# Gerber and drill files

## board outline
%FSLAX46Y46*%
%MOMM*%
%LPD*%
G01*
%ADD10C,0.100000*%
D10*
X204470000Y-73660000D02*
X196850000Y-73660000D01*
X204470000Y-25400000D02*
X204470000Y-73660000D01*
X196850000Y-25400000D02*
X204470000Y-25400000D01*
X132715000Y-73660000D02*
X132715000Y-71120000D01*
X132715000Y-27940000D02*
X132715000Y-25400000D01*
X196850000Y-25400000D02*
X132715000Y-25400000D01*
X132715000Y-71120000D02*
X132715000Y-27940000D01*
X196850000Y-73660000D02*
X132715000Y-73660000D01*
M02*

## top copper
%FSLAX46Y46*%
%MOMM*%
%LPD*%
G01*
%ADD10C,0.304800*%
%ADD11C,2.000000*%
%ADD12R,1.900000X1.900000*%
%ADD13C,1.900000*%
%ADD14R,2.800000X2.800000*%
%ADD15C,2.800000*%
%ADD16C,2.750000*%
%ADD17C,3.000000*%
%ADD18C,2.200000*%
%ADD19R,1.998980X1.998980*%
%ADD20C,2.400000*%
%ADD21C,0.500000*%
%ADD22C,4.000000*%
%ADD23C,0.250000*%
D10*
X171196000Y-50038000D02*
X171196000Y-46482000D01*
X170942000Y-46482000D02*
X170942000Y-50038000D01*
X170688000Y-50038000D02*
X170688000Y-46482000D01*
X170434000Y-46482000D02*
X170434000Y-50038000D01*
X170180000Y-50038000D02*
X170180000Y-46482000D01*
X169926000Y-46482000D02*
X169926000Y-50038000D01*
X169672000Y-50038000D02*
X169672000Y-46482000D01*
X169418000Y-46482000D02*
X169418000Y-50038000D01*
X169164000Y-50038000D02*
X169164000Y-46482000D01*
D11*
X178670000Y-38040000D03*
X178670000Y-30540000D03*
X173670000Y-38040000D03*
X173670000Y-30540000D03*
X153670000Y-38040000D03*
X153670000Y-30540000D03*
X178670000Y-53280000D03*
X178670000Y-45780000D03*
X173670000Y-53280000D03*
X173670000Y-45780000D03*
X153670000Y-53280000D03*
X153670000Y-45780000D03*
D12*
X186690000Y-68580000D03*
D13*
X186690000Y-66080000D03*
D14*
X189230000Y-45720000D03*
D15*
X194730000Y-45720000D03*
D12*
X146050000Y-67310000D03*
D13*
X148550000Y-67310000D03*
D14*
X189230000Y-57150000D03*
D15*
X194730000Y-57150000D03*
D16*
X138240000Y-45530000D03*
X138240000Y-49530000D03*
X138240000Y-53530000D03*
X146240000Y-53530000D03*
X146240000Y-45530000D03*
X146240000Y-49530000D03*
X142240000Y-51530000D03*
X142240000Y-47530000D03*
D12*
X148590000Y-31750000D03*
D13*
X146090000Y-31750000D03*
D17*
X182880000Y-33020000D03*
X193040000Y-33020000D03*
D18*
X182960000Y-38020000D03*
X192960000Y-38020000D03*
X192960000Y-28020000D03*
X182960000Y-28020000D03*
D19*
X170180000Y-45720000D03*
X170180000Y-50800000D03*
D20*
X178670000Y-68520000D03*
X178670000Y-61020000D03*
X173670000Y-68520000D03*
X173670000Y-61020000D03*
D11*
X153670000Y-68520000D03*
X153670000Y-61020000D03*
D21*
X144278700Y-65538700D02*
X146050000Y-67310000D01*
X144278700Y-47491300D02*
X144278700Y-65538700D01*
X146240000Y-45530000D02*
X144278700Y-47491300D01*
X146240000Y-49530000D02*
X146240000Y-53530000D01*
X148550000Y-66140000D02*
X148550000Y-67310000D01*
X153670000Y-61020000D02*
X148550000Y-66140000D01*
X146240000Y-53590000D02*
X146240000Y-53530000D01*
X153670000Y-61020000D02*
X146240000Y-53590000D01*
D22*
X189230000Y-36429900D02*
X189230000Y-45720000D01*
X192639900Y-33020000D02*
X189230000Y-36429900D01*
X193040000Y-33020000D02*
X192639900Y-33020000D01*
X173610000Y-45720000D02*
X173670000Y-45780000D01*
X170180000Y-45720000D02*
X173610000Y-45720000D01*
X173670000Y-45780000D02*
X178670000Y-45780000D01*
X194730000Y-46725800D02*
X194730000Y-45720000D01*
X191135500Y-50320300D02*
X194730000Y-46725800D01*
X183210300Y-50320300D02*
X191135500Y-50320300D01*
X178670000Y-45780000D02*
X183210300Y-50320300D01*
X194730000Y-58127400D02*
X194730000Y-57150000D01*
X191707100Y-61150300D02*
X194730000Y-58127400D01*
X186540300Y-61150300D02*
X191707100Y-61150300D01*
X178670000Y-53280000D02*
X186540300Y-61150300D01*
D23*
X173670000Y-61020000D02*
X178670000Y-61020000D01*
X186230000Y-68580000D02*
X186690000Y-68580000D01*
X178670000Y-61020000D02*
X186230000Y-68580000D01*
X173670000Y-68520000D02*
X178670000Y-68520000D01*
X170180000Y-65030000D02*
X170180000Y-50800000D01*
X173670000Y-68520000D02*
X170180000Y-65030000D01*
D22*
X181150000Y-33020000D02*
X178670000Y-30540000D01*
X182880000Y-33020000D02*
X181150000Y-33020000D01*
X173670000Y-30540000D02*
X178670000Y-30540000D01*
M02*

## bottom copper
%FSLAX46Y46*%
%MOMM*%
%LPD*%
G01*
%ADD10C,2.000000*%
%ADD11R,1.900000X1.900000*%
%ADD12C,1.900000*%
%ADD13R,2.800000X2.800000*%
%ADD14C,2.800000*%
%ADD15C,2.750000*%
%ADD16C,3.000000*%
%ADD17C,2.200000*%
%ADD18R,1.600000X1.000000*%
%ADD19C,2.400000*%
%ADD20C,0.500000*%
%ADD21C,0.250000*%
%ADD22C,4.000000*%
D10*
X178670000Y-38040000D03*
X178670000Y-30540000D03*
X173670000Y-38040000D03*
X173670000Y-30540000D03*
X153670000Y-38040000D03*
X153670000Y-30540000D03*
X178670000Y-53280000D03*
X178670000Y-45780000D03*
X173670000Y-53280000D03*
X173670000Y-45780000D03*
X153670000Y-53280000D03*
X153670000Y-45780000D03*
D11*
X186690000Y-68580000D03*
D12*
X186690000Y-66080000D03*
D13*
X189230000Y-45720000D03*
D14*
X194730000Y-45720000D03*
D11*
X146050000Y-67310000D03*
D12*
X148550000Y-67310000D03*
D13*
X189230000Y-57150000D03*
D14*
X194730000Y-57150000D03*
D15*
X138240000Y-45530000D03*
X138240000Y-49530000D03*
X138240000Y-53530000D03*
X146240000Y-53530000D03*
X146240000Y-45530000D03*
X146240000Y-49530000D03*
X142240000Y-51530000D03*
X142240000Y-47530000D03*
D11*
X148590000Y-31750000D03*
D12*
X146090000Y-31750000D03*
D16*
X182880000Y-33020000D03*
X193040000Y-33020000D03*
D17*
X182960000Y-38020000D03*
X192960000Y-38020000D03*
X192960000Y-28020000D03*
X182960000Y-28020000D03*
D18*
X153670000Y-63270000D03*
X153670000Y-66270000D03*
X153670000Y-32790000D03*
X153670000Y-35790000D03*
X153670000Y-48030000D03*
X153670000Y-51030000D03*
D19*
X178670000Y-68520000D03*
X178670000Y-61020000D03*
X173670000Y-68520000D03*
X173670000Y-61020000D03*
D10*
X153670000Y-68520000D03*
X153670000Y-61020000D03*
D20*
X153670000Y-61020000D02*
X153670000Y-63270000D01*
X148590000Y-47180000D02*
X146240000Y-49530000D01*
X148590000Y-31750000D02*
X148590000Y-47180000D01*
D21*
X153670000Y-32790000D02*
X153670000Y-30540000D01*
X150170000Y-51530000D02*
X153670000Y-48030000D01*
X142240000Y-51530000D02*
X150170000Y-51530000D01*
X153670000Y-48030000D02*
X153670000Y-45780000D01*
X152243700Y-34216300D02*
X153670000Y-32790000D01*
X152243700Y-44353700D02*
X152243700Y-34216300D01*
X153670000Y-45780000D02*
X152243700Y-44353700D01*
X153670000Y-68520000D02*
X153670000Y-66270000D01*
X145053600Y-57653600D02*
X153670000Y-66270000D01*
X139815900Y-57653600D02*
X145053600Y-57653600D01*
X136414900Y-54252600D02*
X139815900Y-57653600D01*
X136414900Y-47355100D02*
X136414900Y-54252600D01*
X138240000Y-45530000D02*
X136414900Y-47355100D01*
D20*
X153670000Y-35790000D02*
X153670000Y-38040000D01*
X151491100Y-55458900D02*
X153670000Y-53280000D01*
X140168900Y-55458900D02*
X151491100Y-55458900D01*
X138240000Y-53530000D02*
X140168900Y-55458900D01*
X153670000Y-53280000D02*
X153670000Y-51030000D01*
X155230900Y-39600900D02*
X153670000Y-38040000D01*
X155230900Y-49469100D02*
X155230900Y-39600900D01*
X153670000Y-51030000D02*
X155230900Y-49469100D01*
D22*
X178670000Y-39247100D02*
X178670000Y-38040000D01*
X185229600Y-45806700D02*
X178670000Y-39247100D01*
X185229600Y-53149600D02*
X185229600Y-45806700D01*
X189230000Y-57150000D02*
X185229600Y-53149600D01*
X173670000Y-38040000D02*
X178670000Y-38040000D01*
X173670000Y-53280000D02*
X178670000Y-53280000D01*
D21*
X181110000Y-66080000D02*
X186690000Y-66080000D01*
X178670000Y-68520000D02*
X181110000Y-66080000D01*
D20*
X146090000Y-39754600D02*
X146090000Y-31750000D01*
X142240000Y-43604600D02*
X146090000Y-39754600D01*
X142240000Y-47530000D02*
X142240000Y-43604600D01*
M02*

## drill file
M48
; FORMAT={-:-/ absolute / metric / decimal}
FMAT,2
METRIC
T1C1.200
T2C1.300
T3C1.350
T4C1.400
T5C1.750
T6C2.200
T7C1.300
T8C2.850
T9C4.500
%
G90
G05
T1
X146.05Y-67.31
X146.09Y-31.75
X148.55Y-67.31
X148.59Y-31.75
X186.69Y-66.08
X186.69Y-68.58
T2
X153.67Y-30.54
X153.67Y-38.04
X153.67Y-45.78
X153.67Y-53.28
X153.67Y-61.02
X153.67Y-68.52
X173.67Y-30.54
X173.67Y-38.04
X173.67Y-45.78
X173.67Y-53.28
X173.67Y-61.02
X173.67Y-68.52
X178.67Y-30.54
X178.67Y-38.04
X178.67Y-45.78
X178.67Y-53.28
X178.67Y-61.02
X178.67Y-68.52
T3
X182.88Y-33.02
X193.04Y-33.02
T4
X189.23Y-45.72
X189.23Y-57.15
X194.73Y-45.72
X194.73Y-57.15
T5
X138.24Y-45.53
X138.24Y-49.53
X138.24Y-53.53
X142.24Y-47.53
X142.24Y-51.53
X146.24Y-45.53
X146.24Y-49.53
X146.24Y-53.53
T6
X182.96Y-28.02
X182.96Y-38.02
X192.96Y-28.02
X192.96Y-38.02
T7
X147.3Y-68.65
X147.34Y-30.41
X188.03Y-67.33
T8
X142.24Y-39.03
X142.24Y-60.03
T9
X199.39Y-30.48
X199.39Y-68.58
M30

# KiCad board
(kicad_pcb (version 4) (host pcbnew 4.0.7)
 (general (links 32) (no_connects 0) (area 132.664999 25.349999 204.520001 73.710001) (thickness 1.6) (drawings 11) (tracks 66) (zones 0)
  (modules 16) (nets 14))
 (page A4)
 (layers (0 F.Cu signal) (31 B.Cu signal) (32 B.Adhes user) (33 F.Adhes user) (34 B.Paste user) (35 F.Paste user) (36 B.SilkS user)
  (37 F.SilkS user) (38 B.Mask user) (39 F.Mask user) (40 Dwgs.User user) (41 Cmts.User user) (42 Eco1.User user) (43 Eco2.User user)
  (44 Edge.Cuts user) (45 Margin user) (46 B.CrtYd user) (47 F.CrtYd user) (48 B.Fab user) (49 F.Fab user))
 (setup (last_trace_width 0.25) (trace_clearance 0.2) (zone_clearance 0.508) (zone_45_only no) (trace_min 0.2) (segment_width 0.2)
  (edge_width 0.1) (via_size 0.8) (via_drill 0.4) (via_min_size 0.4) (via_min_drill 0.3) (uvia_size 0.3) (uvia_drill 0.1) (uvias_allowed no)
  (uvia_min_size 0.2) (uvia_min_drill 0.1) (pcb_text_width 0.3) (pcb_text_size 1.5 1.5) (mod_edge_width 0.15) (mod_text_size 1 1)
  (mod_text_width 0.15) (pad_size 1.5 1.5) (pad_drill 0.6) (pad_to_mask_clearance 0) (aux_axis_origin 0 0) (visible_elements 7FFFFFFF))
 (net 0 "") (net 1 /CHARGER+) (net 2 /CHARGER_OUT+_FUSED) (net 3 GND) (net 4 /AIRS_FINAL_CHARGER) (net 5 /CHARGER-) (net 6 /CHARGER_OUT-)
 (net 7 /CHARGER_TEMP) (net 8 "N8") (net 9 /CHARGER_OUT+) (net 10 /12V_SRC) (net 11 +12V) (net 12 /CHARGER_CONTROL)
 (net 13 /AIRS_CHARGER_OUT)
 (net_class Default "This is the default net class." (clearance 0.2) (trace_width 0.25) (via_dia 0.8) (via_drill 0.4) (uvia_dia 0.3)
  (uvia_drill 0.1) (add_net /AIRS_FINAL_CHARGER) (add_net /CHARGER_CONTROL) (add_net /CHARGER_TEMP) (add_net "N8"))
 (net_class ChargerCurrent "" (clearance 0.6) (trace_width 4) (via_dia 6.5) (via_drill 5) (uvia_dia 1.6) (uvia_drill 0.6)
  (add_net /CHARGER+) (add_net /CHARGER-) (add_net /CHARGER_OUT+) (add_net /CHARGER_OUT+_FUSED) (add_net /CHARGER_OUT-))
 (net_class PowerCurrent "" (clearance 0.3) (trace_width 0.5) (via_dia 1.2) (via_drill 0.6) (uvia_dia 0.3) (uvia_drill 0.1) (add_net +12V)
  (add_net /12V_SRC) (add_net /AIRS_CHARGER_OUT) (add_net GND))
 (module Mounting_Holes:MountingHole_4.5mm (layer F.Cu) (at 199.39 68.58)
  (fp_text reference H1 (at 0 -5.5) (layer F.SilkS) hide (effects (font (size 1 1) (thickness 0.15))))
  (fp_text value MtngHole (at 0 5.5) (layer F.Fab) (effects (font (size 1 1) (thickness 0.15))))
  (pad 1 np_thru_hole circle (at 0 0) (size 4.5 4.5) (drill 4.5) (layers *.Cu *.Mask)))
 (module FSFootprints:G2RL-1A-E (layer F.Cu) (at 153.67 34.29)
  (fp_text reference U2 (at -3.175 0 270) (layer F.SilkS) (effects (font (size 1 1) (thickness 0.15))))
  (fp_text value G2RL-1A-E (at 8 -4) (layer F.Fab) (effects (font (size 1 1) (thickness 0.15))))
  (pad 5 thru_hole circle (at 25 3.75) (size 2 2) (drill 1.3) (layers *.Cu *.Mask) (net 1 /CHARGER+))
  (pad 4 thru_hole circle (at 25 -3.75) (size 2 2) (drill 1.3) (layers *.Cu *.Mask) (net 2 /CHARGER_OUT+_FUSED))
  (pad 6 thru_hole circle (at 20 3.75) (size 2 2) (drill 1.3) (layers *.Cu *.Mask) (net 1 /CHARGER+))
  (pad 3 thru_hole circle (at 20 -3.75) (size 2 2) (drill 1.3) (layers *.Cu *.Mask) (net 2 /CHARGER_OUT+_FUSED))
  (pad 8 thru_hole circle (at 0 3.75) (size 2 2) (drill 1.3) (layers *.Cu *.Mask) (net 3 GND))
  (pad 1 thru_hole circle (at 0 -3.75) (size 2 2) (drill 1.3) (layers *.Cu *.Mask) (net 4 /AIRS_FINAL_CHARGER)))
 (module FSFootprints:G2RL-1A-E (layer F.Cu) (at 153.67 49.53)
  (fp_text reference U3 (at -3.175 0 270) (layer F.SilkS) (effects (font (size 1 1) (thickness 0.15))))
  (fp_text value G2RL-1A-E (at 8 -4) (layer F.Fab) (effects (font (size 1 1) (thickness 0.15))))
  (pad 5 thru_hole circle (at 25 3.75) (size 2 2) (drill 1.3) (layers *.Cu *.Mask) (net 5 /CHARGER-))
  (pad 4 thru_hole circle (at 25 -3.75) (size 2 2) (drill 1.3) (layers *.Cu *.Mask) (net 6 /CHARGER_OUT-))
  (pad 6 thru_hole circle (at 20 3.75) (size 2 2) (drill 1.3) (layers *.Cu *.Mask) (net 5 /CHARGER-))
  (pad 3 thru_hole circle (at 20 -3.75) (size 2 2) (drill 1.3) (layers *.Cu *.Mask) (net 6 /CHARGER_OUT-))
  (pad 8 thru_hole circle (at 0 3.75) (size 2 2) (drill 1.3) (layers *.Cu *.Mask) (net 3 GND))
  (pad 1 thru_hole circle (at 0 -3.75) (size 2 2) (drill 1.3) (layers *.Cu *.Mask) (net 4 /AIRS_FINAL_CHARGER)))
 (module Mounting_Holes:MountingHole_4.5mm (layer F.Cu) (at 199.39 30.48 180)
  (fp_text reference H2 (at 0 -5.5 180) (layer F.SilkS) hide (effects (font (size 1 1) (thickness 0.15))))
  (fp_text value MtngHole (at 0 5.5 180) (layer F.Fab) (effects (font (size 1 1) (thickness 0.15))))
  (pad 1 np_thru_hole circle (at 0 0 180) (size 4.5 4.5) (drill 4.5) (layers *.Cu *.Mask)))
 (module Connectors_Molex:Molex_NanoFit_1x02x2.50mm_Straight (layer F.Cu) (at 186.69 68.58 90)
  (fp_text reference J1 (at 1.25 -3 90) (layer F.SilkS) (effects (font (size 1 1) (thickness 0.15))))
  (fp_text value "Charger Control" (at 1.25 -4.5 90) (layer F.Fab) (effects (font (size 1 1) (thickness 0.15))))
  (pad 1 thru_hole rect (at 0 0 90) (size 1.9 1.9) (drill 1.2) (layers *.Cu *.Mask) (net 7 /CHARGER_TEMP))
  (pad 2 thru_hole circle (at 2.5 0 90) (size 1.9 1.9) (drill 1.2) (layers *.Cu *.Mask) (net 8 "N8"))
  (pad "" np_thru_hole circle (at 1.25 1.34 90) (size 1.3 1.3) (drill 1.3) (layers *.Cu *.Mask)))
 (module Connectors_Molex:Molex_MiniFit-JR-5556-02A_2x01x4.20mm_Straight (layer F.Cu) (at 189.23 45.72 90)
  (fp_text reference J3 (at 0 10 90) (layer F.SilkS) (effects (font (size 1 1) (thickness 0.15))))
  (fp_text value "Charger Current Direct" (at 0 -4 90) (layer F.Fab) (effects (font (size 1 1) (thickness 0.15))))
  (pad 1 thru_hole rect (at 0 0 90) (size 2.8 2.8) (drill 1.4) (layers *.Cu *.Mask) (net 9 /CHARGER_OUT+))
  (pad 2 thru_hole circle (at 0 5.5 90) (size 2.8 2.8) (drill 1.4) (layers *.Cu *.Mask) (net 6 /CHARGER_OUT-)))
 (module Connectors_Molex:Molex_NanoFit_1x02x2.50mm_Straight (layer F.Cu) (at 146.05 67.31)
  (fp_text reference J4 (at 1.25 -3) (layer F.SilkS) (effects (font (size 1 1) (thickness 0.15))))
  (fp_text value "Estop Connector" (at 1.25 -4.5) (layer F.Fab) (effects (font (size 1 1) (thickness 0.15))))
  (pad 1 thru_hole rect (at 0 0) (size 1.9 1.9) (drill 1.2) (layers *.Cu *.Mask) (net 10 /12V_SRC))
  (pad 2 thru_hole circle (at 2.5 0) (size 1.9 1.9) (drill 1.2) (layers *.Cu *.Mask) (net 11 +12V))
  (pad "" np_thru_hole circle (at 1.25 1.34) (size 1.3 1.3) (drill 1.3) (layers *.Cu *.Mask)))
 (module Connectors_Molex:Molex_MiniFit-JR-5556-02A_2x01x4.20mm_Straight (layer F.Cu) (at 189.23 57.15 90)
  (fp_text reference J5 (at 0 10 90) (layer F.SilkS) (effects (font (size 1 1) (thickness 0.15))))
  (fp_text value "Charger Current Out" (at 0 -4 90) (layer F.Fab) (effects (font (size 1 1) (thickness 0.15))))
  (pad 1 thru_hole rect (at 0 0 90) (size 2.8 2.8) (drill 1.4) (layers *.Cu *.Mask) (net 1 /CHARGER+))
  (pad 2 thru_hole circle (at 0 5.5 90) (size 2.8 2.8) (drill 1.4) (layers *.Cu *.Mask) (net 5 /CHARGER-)))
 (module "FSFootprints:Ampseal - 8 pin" (layer F.Cu) (at 142.24 49.53 270)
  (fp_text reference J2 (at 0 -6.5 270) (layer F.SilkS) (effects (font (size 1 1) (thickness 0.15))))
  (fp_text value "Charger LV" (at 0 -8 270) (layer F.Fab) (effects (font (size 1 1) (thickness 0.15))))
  (pad "" np_thru_hole circle (at -10.5 0 270) (size 2.85 2.85) (drill 2.85) (layers *.Cu *.Mask))
  (pad 6 thru_hole circle (at -4 4 270) (size 2.75 2.75) (drill 1.75) (layers *.Cu *.Mask) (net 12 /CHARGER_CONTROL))
  (pad 7 thru_hole circle (at 0 4 270) (size 2.75 2.75) (drill 1.75) (layers *.Cu *.Mask))
  (pad 8 thru_hole circle (at 4 4 270) (size 2.75 2.75) (drill 1.75) (layers *.Cu *.Mask) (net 3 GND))
  (pad 3 thru_hole circle (at 4 -4 270) (size 2.75 2.75) (drill 1.75) (layers *.Cu *.Mask) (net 11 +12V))
  (pad 1 thru_hole circle (at -4 -4 270) (size 2.75 2.75) (drill 1.75) (layers *.Cu *.Mask) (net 10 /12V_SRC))
  (pad 2 thru_hole circle (at 0 -4 270) (size 2.75 2.75) (drill 1.75) (layers *.Cu *.Mask) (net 11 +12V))
  (pad 5 thru_hole circle (at 2 0 270) (size 2.75 2.75) (drill 1.75) (layers *.Cu *.Mask) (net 4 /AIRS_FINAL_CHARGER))
  (pad 4 thru_hole circle (at -2 0 270) (size 2.75 2.75) (drill 1.75) (layers *.Cu *.Mask) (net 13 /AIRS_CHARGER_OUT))
  (pad "" np_thru_hole circle (at 10.5 0 270) (size 2.85 2.85) (drill 2.85) (layers *.Cu *.Mask)))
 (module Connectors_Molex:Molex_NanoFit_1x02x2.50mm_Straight (layer F.Cu) (at 148.59 31.75 180)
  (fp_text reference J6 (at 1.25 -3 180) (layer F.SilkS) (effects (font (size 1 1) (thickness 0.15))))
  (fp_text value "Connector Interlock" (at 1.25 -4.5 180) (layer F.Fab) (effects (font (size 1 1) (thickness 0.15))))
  (pad 1 thru_hole rect (at 0 0 180) (size 1.9 1.9) (drill 1.2) (layers *.Cu *.Mask) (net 11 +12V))
  (pad 2 thru_hole circle (at 2.5 0 180) (size 1.9 1.9) (drill 1.2) (layers *.Cu *.Mask) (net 13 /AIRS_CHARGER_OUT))
  (pad "" np_thru_hole circle (at 1.25 1.34 180) (size 1.3 1.3) (drill 1.3) (layers *.Cu *.Mask)))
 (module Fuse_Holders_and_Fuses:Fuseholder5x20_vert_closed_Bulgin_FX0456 (layer F.Cu) (at 193.04 33.02 180)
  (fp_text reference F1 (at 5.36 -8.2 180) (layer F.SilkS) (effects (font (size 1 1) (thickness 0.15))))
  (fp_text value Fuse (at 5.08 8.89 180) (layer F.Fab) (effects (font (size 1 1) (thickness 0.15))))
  (pad 2 thru_hole circle (at 10.16 0 180) (size 3 3) (drill 1.35) (layers *.Cu *.Mask) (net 2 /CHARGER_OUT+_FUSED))
  (pad 1 thru_hole circle (at 0 0 180) (size 3 3) (drill 1.35) (layers *.Cu *.Mask) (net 9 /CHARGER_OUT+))
  (pad 3 thru_hole circle (at 10.08 -5 180) (size 2.2 2.2) (drill 2.2) (layers *.Cu Dwgs.User))
  (pad 3 thru_hole circle (at 0.08 -5 180) (size 2.2 2.2) (drill 2.2) (layers *.Cu Dwgs.User))
  (pad 3 thru_hole circle (at 0.08 5 180) (size 2.2 2.2) (drill 2.2) (layers *.Cu Dwgs.User))
  (pad 3 thru_hole circle (at 10.08 5 180) (size 2.2 2.2) (drill 2.2) (layers *.Cu Dwgs.User)))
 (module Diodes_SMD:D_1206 (layer B.Cu) (at 153.67 64.77 270)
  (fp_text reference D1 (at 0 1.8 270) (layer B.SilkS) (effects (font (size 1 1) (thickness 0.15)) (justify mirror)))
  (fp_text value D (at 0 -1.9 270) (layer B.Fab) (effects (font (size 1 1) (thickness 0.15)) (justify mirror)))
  (pad 1 smd rect (at -1.5 0 270) (size 1 1.6) (layers B.Cu B.Paste B.Mask) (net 11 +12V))
  (pad 2 smd rect (at 1.5 0 270) (size 1 1.6) (layers B.Cu B.Paste B.Mask) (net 12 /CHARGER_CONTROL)))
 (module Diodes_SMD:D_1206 (layer B.Cu) (at 153.67 34.29 270)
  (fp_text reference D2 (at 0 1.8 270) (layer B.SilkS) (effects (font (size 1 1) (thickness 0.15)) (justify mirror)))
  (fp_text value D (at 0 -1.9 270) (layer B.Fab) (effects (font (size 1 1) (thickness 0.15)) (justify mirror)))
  (pad 1 smd rect (at -1.5 0 270) (size 1 1.6) (layers B.Cu B.Paste B.Mask) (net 4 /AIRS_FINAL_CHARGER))
  (pad 2 smd rect (at 1.5 0 270) (size 1 1.6) (layers B.Cu B.Paste B.Mask) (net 3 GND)))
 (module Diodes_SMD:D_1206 (layer B.Cu) (at 153.67 49.53 270)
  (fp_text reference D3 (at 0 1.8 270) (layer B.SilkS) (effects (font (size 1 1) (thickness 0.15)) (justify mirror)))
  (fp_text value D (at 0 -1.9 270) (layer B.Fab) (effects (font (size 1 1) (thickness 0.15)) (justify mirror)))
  (pad 1 smd rect (at -1.5 0 270) (size 1 1.6) (layers B.Cu B.Paste B.Mask) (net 4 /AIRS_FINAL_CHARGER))
  (pad 2 smd rect (at 1.5 0 270) (size 1 1.6) (layers B.Cu B.Paste B.Mask) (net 3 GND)))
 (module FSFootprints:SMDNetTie (layer F.Cu) (at 170.18 48.26 270)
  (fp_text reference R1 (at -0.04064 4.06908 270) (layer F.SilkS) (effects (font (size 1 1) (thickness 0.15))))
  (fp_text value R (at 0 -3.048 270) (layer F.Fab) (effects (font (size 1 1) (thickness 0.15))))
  (fp_line (start 1.778 -1.016) (end -1.778 -1.016) (layer F.Cu) (width 0.3048))
  (fp_line (start -1.778 -0.762) (end 1.778 -0.762) (layer F.Cu) (width 0.3048))
  (fp_line (start 1.778 -0.508) (end -1.778 -0.508) (layer F.Cu) (width 0.3048))
  (fp_line (start -1.778 -0.254) (end 1.778 -0.254) (layer F.Cu) (width 0.3048))
  (fp_line (start 1.778 0) (end -1.778 0) (layer F.Cu) (width 0.3048))
  (fp_line (start -1.778 0.254) (end 1.778 0.254) (layer F.Cu) (width 0.3048))
  (fp_line (start 1.778 0.508) (end -1.778 0.508) (layer F.Cu) (width 0.3048))
  (fp_line (start -1.778 0.762) (end 1.778 0.762) (layer F.Cu) (width 0.3048))
  (fp_line (start 1.778 1.016) (end -1.778 1.016) (layer F.Cu) (width 0.3048))
  (pad 1 smd rect (at -2.54 0 270) (size 1.99898 1.99898) (layers F.Cu) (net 6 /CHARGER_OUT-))
  (pad 2 smd rect (at 2.54 0 270) (size 1.99898 1.99898) (layers F.Cu) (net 8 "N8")))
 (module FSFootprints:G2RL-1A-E (layer F.Cu) (at 153.67 64.77)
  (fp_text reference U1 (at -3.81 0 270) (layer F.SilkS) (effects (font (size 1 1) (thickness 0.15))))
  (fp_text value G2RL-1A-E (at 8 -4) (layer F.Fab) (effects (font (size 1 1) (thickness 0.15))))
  (pad 5 thru_hole circle (at 25 3.75) (size 2.4 2.4) (drill 1.3) (layers *.Cu *.Mask) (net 8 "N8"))
  (pad 4 thru_hole circle (at 25 -3.75) (size 2.4 2.4) (drill 1.3) (layers *.Cu *.Mask) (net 7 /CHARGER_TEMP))
  (pad 6 thru_hole circle (at 20 3.75) (size 2.4 2.4) (drill 1.3) (layers *.Cu *.Mask) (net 8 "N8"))
  (pad 3 thru_hole circle (at 20 -3.75) (size 2.4 2.4) (drill 1.3) (layers *.Cu *.Mask) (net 7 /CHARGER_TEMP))
  (pad 8 thru_hole circle (at 0 3.75) (size 2 2) (drill 1.3) (layers *.Cu *.Mask) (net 12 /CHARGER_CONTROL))
  (pad 1 thru_hole circle (at 0 -3.75) (size 2 2) (drill 1.3) (layers *.Cu *.Mask) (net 11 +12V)))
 (gr_line (start 204.47 73.66) (end 196.85 73.66) (angle 90) (layer Edge.Cuts) (width 0.1))
 (gr_line (start 204.47 25.4) (end 204.47 73.66) (angle 90) (layer Edge.Cuts) (width 0.1))
 (gr_line (start 196.85 25.4) (end 204.47 25.4) (angle 90) (layer Edge.Cuts) (width 0.1))
 (gr_line (start 132.715 73.66) (end 132.715 71.12) (angle 90) (layer Edge.Cuts) (width 0.1))
 (gr_line (start 132.715 27.94) (end 132.715 25.4) (angle 90) (layer Edge.Cuts) (width 0.1))
 (gr_line (start 196.85 25.4) (end 132.715 25.4) (angle 90) (layer Edge.Cuts) (width 0.1))
 (gr_line (start 132.715 71.12) (end 132.715 27.94) (angle 90) (layer Edge.Cuts) (width 0.1))
 (gr_line (start 196.85 73.66) (end 132.715 73.66) (angle 90) (layer Edge.Cuts) (width 0.1))
 (segment (start 144.2787 65.5387) (end 146.05 67.31) (width 0.5) (layer F.Cu) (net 10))
 (segment (start 144.2787 47.4913) (end 144.2787 65.5387) (width 0.5) (layer F.Cu) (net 10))
 (segment (start 146.24 45.53) (end 144.2787 47.4913) (width 0.5) (layer F.Cu) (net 10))
 (segment (start 153.67 61.02) (end 153.67 63.27) (width 0.5) (layer B.Cu) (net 11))
 (segment (start 146.24 49.53) (end 146.24 53.53) (width 0.5) (layer F.Cu) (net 11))
 (segment (start 148.59 47.18) (end 146.24 49.53) (width 0.5) (layer B.Cu) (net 11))
 (segment (start 148.59 31.75) (end 148.59 47.18) (width 0.5) (layer B.Cu) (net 11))
 (segment (start 148.55 66.14) (end 148.55 67.31) (width 0.5) (layer F.Cu) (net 11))
 (segment (start 153.67 61.02) (end 148.55 66.14) (width 0.5) (layer F.Cu) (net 11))
 (segment (start 146.24 53.59) (end 146.24 53.53) (width 0.5) (layer F.Cu) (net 11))
 (segment (start 153.67 61.02) (end 146.24 53.59) (width 0.5) (layer F.Cu) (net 11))
 (segment (start 153.67 32.79) (end 153.67 30.54) (width 0.25) (layer B.Cu) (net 4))
 (segment (start 150.17 51.53) (end 153.67 48.03) (width 0.25) (layer B.Cu) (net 4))
 (segment (start 142.24 51.53) (end 150.17 51.53) (width 0.25) (layer B.Cu) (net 4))
 (segment (start 153.67 48.03) (end 153.67 45.78) (width 0.25) (layer B.Cu) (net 4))
 (segment (start 152.2437 34.2163) (end 153.67 32.79) (width 0.25) (layer B.Cu) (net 4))
 (segment (start 152.2437 44.3537) (end 152.2437 34.2163) (width 0.25) (layer B.Cu) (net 4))
 (segment (start 153.67 45.78) (end 152.2437 44.3537) (width 0.25) (layer B.Cu) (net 4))
 (segment (start 153.67 68.52) (end 153.67 66.27) (width 0.25) (layer B.Cu) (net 12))
 (segment (start 145.0536 57.6536) (end 153.67 66.27) (width 0.25) (layer B.Cu) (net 12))
 (segment (start 139.8159 57.6536) (end 145.0536 57.6536) (width 0.25) (layer B.Cu) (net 12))
 (segment (start 136.4149 54.2526) (end 139.8159 57.6536) (width 0.25) (layer B.Cu) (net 12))
 (segment (start 136.4149 47.3551) (end 136.4149 54.2526) (width 0.25) (layer B.Cu) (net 12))
 (segment (start 138.24 45.53) (end 136.4149 47.3551) (width 0.25) (layer B.Cu) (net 12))
 (segment (start 153.67 35.79) (end 153.67 38.04) (width 0.5) (layer B.Cu) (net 3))
 (segment (start 151.4911 55.4589) (end 153.67 53.28) (width 0.5) (layer B.Cu) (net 3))
 (segment (start 140.1689 55.4589) (end 151.4911 55.4589) (width 0.5) (layer B.Cu) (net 3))
 (segment (start 138.24 53.53) (end 140.1689 55.4589) (width 0.5) (layer B.Cu) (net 3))
 (segment (start 153.67 53.28) (end 153.67 51.03) (width 0.5) (layer B.Cu) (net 3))
 (segment (start 155.2309 39.6009) (end 153.67 38.04) (width 0.5) (layer B.Cu) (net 3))
 (segment (start 155.2309 49.4691) (end 155.2309 39.6009) (width 0.5) (layer B.Cu) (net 3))
 (segment (start 153.67 51.03) (end 155.2309 49.4691) (width 0.5) (layer B.Cu) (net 3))
 (segment (start 189.23 36.4299) (end 189.23 45.72) (width 4) (layer F.Cu) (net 9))
 (segment (start 192.6399 33.02) (end 189.23 36.4299) (width 4) (layer F.Cu) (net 9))
 (segment (start 193.04 33.02) (end 192.6399 33.02) (width 4) (layer F.Cu) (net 9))
 (segment (start 173.61 45.72) (end 173.67 45.78) (width 4) (layer F.Cu) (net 6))
 (segment (start 170.18 45.72) (end 173.61 45.72) (width 4) (layer F.Cu) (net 6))
 (segment (start 173.67 45.78) (end 178.67 45.78) (width 4) (layer F.Cu) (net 6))
 (segment (start 194.73 46.7258) (end 194.73 45.72) (width 4) (layer F.Cu) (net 6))
 (segment (start 191.1355 50.3203) (end 194.73 46.7258) (width 4) (layer F.Cu) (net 6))
 (segment (start 183.2103 50.3203) (end 191.1355 50.3203) (width 4) (layer F.Cu) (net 6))
 (segment (start 178.67 45.78) (end 183.2103 50.3203) (width 4) (layer F.Cu) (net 6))
 (segment (start 178.67 39.2471) (end 178.67 38.04) (width 4) (layer B.Cu) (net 1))
 (segment (start 185.2296 45.8067) (end 178.67 39.2471) (width 4) (layer B.Cu) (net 1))
 (segment (start 185.2296 53.1496) (end 185.2296 45.8067) (width 4) (layer B.Cu) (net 1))
 (segment (start 189.23 57.15) (end 185.2296 53.1496) (width 4) (layer B.Cu) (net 1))
 (segment (start 173.67 38.04) (end 178.67 38.04) (width 4) (layer B.Cu) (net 1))
 (segment (start 194.73 58.1274) (end 194.73 57.15) (width 4) (layer F.Cu) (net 5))
 (segment (start 191.7071 61.1503) (end 194.73 58.1274) (width 4) (layer F.Cu) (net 5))
 (segment (start 186.5403 61.1503) (end 191.7071 61.1503) (width 4) (layer F.Cu) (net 5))
 (segment (start 178.67 53.28) (end 186.5403 61.1503) (width 4) (layer F.Cu) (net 5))
 (segment (start 173.67 53.28) (end 178.67 53.28) (width 4) (layer B.Cu) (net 5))
 (segment (start 173.67 61.02) (end 178.67 61.02) (width 0.25) (layer F.Cu) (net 7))
 (segment (start 186.23 68.58) (end 186.69 68.58) (width 0.25) (layer F.Cu) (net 7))
 (segment (start 178.67 61.02) (end 186.23 68.58) (width 0.25) (layer F.Cu) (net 7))
 (segment (start 181.11 66.08) (end 186.69 66.08) (width 0.25) (layer B.Cu) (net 8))
 (segment (start 178.67 68.52) (end 181.11 66.08) (width 0.25) (layer B.Cu) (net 8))
 (segment (start 173.67 68.52) (end 178.67 68.52) (width 0.25) (layer F.Cu) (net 8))
 (segment (start 170.18 65.03) (end 170.18 50.8) (width 0.25) (layer F.Cu) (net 8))
 (segment (start 173.67 68.52) (end 170.18 65.03) (width 0.25) (layer F.Cu) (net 8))
 (segment (start 146.09 39.7546) (end 146.09 31.75) (width 0.5) (layer B.Cu) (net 13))
 (segment (start 142.24 43.6046) (end 146.09 39.7546) (width 0.5) (layer B.Cu) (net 13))
 (segment (start 142.24 47.53) (end 142.24 43.6046) (width 0.5) (layer B.Cu) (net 13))
 (segment (start 181.15 33.02) (end 178.67 30.54) (width 4) (layer F.Cu) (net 2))
 (segment (start 182.88 33.02) (end 181.15 33.02) (width 4) (layer F.Cu) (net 2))
 (segment (start 173.67 30.54) (end 178.67 30.54) (width 4) (layer F.Cu) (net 2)))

